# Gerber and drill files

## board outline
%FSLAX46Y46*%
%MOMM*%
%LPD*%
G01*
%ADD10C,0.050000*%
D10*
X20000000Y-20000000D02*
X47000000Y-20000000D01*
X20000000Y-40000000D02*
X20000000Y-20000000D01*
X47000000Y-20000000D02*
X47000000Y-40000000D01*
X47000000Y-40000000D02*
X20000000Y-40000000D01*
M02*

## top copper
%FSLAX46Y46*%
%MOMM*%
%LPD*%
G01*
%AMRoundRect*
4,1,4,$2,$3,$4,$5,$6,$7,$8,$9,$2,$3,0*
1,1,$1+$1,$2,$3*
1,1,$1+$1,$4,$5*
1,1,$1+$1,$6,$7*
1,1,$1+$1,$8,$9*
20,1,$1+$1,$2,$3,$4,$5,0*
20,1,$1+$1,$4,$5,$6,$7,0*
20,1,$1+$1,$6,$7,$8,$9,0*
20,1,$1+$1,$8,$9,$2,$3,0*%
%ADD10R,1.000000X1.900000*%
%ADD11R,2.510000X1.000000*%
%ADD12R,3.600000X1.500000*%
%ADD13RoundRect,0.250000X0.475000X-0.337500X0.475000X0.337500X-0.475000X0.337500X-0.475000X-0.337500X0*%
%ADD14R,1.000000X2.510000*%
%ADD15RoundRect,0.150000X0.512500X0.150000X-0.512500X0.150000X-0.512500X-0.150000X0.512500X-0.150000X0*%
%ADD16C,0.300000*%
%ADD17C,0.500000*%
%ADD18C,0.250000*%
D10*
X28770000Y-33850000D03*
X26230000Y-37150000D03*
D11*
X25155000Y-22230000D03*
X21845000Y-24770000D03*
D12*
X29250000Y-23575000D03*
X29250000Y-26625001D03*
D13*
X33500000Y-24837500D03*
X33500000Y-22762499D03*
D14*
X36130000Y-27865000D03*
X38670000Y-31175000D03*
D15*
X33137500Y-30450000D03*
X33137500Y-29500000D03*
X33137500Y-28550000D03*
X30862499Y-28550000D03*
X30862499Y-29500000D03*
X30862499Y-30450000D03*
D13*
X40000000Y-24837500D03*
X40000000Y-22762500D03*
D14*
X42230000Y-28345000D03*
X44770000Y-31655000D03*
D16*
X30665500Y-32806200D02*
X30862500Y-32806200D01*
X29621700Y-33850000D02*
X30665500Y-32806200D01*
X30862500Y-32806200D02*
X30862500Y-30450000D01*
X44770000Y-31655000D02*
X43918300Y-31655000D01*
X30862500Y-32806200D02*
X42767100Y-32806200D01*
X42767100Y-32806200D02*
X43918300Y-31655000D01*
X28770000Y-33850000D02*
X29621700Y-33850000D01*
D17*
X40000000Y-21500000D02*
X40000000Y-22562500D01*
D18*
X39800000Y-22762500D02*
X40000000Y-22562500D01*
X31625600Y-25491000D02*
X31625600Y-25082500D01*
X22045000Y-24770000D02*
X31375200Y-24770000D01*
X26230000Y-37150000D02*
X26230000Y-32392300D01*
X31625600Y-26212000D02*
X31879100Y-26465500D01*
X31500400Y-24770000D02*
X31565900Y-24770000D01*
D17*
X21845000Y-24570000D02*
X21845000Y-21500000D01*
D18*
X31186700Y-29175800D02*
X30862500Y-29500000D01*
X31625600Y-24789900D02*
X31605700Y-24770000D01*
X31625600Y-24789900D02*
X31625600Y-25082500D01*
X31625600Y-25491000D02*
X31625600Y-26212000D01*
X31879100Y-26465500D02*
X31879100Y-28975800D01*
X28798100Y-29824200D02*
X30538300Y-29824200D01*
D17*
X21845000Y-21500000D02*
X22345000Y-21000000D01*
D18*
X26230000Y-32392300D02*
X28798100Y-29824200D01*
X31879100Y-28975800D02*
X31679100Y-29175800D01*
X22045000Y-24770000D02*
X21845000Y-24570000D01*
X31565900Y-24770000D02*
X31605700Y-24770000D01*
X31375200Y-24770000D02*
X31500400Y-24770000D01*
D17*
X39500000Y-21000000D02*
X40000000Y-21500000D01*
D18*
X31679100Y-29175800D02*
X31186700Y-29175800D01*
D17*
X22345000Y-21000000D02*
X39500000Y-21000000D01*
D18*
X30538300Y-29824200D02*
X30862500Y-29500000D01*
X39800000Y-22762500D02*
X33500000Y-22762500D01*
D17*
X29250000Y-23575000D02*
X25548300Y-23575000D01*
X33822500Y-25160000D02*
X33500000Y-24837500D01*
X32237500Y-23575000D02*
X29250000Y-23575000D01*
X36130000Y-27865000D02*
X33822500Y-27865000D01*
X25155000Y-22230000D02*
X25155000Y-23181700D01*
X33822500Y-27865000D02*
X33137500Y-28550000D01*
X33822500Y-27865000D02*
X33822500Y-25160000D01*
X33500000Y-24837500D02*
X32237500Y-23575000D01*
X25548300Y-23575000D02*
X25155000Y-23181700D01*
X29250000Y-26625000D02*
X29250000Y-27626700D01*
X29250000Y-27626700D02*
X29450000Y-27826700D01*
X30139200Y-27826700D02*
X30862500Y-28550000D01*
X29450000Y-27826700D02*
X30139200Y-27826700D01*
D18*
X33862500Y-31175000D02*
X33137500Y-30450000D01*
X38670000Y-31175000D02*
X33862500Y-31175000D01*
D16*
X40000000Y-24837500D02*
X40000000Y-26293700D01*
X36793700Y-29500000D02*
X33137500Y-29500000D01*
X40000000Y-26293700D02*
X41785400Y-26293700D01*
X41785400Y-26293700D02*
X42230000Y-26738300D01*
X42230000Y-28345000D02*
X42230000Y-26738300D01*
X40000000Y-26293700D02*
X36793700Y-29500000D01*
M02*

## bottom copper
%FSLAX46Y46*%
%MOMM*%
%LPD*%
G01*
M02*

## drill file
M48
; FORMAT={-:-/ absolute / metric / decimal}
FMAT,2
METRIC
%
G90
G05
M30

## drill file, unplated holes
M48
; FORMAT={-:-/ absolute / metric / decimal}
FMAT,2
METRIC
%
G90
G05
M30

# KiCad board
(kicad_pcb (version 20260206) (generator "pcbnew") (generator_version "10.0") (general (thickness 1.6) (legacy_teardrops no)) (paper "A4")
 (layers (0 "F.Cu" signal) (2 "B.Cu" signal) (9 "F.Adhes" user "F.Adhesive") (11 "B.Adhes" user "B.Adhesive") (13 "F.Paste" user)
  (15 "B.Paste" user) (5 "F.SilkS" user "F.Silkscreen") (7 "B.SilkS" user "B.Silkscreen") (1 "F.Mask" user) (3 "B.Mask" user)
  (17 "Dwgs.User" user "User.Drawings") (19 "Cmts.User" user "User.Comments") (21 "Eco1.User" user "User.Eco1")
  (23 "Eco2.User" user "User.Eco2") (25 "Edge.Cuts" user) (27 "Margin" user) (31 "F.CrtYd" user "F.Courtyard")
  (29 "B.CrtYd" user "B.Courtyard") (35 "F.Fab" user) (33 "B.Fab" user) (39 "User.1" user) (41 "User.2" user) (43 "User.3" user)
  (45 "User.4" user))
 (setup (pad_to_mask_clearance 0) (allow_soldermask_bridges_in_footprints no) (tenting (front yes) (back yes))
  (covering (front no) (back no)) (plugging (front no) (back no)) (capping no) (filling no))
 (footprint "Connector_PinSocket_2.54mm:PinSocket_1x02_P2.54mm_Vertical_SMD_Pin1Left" (layer "F.Cu") (at 27.5 35.5 -90)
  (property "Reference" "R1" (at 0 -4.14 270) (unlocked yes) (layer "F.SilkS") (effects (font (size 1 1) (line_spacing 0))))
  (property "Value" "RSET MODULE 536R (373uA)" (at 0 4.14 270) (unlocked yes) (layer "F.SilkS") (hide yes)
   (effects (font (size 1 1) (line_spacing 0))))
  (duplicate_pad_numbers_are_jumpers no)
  (pad "1" smd rect (at -1.65 -1.27 270) (size 1.9 1) (layers "F.Cu" "F.Mask" "F.Paste") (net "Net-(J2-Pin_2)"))
  (pad "2" smd rect (at 1.65 1.27 270) (size 1.9 1) (layers "F.Cu" "F.Mask" "F.Paste") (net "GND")))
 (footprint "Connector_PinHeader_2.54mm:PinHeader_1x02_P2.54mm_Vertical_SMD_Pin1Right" (layer "F.Cu") (at 23.5 23.5)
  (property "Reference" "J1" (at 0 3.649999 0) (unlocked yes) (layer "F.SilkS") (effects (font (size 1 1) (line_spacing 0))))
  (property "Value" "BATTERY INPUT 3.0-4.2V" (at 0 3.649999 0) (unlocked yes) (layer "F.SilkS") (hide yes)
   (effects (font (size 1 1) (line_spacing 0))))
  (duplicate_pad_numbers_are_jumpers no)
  (pad "1" smd rect (at 1.655 -1.27) (size 2.51 1) (layers "F.Cu" "F.Mask" "F.Paste") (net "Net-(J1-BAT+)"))
  (pad "2" smd rect (at -1.655 1.27) (size 2.51 1) (layers "F.Cu" "F.Mask" "F.Paste") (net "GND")))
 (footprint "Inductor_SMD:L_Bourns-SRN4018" (layer "F.Cu") (at 29.25 25.1 -90)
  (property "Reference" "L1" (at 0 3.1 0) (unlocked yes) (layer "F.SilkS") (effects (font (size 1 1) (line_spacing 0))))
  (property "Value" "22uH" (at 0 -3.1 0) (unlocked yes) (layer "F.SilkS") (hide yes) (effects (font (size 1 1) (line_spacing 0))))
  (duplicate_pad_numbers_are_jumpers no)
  (pad "1" smd rect (at -1.525 0 270) (size 1.5 3.6) (layers "F.Cu" "F.Mask" "F.Paste") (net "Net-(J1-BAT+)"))
  (pad "2" smd rect (at 1.525001 0 270) (size 1.5 3.6) (layers "F.Cu" "F.Mask" "F.Paste") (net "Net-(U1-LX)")))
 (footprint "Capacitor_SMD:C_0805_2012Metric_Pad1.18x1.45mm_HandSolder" (layer "F.Cu") (at 33.5 23.8 90)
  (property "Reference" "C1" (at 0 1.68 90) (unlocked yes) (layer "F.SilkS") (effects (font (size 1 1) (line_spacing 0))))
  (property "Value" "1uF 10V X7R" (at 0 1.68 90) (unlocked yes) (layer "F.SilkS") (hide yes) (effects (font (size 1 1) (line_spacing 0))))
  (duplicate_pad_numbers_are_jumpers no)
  (pad "1" smd roundrect (at -1.0375 0 90) (size 1.175 1.45) (layers "F.Cu" "F.Mask" "F.Paste") (roundrect_rratio 0.212766)
   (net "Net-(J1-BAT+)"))
  (pad "2" smd roundrect (at 1.037501 0 90) (size 1.175 1.45) (layers "F.Cu" "F.Mask" "F.Paste") (roundrect_rratio 0.212766) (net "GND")
   (zone_connect 3)))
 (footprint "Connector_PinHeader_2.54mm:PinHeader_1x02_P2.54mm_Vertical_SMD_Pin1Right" (layer "F.Cu") (at 37.4 29.52 90)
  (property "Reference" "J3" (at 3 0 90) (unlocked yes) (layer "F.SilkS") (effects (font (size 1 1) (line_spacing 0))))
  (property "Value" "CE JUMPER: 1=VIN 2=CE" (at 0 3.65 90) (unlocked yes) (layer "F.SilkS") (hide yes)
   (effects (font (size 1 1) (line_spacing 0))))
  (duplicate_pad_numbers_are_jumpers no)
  (pad "1" smd rect (at 1.655 -1.27 90) (size 2.51 1) (layers "F.Cu" "F.Mask" "F.Paste") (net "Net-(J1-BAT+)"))
  (pad "2" smd rect (at -1.655 1.27 90) (size 2.51 1) (layers "F.Cu" "F.Mask" "F.Paste") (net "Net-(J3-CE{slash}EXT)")))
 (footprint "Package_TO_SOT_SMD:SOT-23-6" (layer "F.Cu") (at 32 29.5 180)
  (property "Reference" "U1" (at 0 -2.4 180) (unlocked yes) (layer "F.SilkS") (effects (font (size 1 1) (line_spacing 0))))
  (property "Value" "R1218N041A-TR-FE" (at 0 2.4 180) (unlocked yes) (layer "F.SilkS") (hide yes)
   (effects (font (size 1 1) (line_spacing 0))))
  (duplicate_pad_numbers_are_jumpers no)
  (pad "1" smd roundrect (at -1.1375 -0.95 180) (size 1.325 0.6) (layers "F.Cu" "F.Mask" "F.Paste") (roundrect_rratio 0.25)
   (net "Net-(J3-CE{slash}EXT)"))
  (pad "2" smd roundrect (at -1.1375 0 180) (size 1.325 0.6) (layers "F.Cu" "F.Mask" "F.Paste") (roundrect_rratio 0.25)
   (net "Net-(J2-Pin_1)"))
  (pad "3" smd roundrect (at -1.1375 0.95 180) (size 1.325 0.6) (layers "F.Cu" "F.Mask" "F.Paste") (roundrect_rratio 0.25)
   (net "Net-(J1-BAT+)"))
  (pad "4" smd roundrect (at 1.137501 0.95 180) (size 1.325 0.6) (layers "F.Cu" "F.Mask" "F.Paste") (roundrect_rratio 0.25)
   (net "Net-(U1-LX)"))
  (pad "5" smd roundrect (at 1.137501 0 180) (size 1.325 0.6) (layers "F.Cu" "F.Mask" "F.Paste") (roundrect_rratio 0.25) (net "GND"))
  (pad "6" smd roundrect (at 1.137501 -0.95 180) (size 1.325 0.6) (layers "F.Cu" "F.Mask" "F.Paste") (roundrect_rratio 0.25)
   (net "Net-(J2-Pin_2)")))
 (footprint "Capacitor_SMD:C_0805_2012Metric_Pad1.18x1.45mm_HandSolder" (layer "F.Cu") (at 40 23.8 90)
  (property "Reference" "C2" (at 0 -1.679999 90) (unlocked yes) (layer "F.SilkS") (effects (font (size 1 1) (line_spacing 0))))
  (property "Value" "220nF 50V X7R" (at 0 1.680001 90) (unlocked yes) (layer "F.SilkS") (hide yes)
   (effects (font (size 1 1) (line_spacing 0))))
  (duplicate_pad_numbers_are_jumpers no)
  (pad "1" smd roundrect (at -1.0375 0 90) (size 1.175 1.45) (layers "F.Cu" "F.Mask" "F.Paste") (roundrect_rratio 0.212766)
   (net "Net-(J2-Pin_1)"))
  (pad "2" smd roundrect (at 1.0375 0 90) (size 1.175 1.45) (layers "F.Cu" "F.Mask" "F.Paste") (roundrect_rratio 0.212766) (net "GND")
   (zone_connect 3)))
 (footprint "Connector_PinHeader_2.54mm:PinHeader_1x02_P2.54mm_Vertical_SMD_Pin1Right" (layer "F.Cu") (at 43.5 30 90)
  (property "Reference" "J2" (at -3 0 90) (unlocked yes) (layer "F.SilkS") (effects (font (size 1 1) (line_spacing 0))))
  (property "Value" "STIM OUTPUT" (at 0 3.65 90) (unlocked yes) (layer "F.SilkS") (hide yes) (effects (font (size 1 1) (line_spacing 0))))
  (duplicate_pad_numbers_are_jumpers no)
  (pad "1" smd rect (at 1.655 -1.27 90) (size 2.51 1) (layers "F.Cu" "F.Mask" "F.Paste") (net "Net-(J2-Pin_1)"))
  (pad "2" smd rect (at -1.655 1.27 90) (size 2.51 1) (layers "F.Cu" "F.Mask" "F.Paste") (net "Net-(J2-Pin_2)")))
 (gr_line (start 20 20) (end 47 20) (stroke (width 0.05) (type default)) (layer "Edge.Cuts"))
 (gr_line (start 20 40) (end 20 20) (stroke (width 0.05) (type default)) (layer "Edge.Cuts"))
 (gr_line (start 47 20) (end 47 40) (stroke (width 0.05) (type default)) (layer "Edge.Cuts"))
 (gr_line (start 47 40) (end 20 40) (stroke (width 0.05) (type default)) (layer "Edge.Cuts"))
 (segment (start 30.6655 32.8062) (end 30.8625 32.8062) (width 0.3) (layer "F.Cu") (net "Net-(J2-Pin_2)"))
 (segment (start 29.6217 33.85) (end 30.6655 32.8062) (width 0.3) (layer "F.Cu") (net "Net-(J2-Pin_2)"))
 (segment (start 30.8625 32.8062) (end 30.8625 30.45) (width 0.3) (layer "F.Cu") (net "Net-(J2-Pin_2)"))
 (segment (start 44.77 31.655) (end 43.9183 31.655) (width 0.3) (layer "F.Cu") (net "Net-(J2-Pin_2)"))
 (segment (start 30.8625 32.8062) (end 42.7671 32.8062) (width 0.3) (layer "F.Cu") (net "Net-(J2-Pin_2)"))
 (segment (start 42.7671 32.8062) (end 43.9183 31.655) (width 0.3) (layer "F.Cu") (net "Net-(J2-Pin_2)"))
 (segment (start 28.77 33.85) (end 29.6217 33.85) (width 0.3) (layer "F.Cu") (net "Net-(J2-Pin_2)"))
 (segment (start 31.6256 25.491) (end 31.6256 25.0825) (width 0.25) (layer "F.Cu") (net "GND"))
 (segment (start 22.045000 24.770000) (end 31.3752 24.77) (width 0.25) (layer "F.Cu") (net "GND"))
 (segment (start 26.23 37.15) (end 26.23 32.3923) (width 0.25) (layer "F.Cu") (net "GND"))
 (segment (start 31.6256 26.212) (end 31.8791 26.4655) (width 0.25) (layer "F.Cu") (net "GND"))
 (segment (start 31.5004 24.77) (end 31.5659 24.77) (width 0.25) (layer "F.Cu") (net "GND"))
 (segment (start 31.1867 29.1758) (end 30.8625 29.5) (width 0.25) (layer "F.Cu") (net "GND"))
 (segment (start 31.625600 24.789900) (end 31.6256 25.0825) (width 0.25) (layer "F.Cu") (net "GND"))
 (segment (start 31.6256 25.491) (end 31.6256 26.212) (width 0.25) (layer "F.Cu") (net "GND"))
 (segment (start 31.8791 26.4655) (end 31.879100 28.975800) (width 0.25) (layer "F.Cu") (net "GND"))
 (segment (start 28.7981 29.8242) (end 30.5383 29.8242) (width 0.25) (layer "F.Cu") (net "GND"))
 (segment (start 26.23 32.3923) (end 28.7981 29.8242) (width 0.25) (layer "F.Cu") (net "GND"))
 (segment (start 31.5659 24.77) (end 31.605700 24.770000) (width 0.25) (layer "F.Cu") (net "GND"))
 (segment (start 31.3752 24.77) (end 31.5004 24.77) (width 0.25) (layer "F.Cu") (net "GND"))
 (segment (start 31.679100 29.175800) (end 31.1867 29.1758) (width 0.25) (layer "F.Cu") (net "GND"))
 (segment (start 30.5383 29.8242) (end 30.8625 29.5) (width 0.25) (layer "F.Cu") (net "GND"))
 (segment (start 39.800000 22.762500) (end 33.5 22.7625) (width 0.25) (layer "F.Cu") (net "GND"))
 (segment (start 29.25 23.575) (end 25.5483 23.575) (width 0.5) (layer "F.Cu") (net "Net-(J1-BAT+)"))
 (segment (start 33.8225 25.16) (end 33.5 24.8375) (width 0.5) (layer "F.Cu") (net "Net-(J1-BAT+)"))
 (segment (start 32.2375 23.575) (end 29.25 23.575) (width 0.5) (layer "F.Cu") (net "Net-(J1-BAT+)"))
 (segment (start 36.13 27.865) (end 33.8225 27.865) (width 0.5) (layer "F.Cu") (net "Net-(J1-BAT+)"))
 (segment (start 25.155 22.23) (end 25.155 23.1817) (width 0.5) (layer "F.Cu") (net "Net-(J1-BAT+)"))
 (segment (start 33.8225 27.865) (end 33.1375 28.55) (width 0.5) (layer "F.Cu") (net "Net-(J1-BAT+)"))
 (segment (start 33.8225 27.865) (end 33.8225 25.16) (width 0.5) (layer "F.Cu") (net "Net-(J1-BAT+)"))
 (segment (start 33.5 24.8375) (end 32.2375 23.575) (width 0.5) (layer "F.Cu") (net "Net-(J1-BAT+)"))
 (segment (start 25.5483 23.575) (end 25.155 23.1817) (width 0.5) (layer "F.Cu") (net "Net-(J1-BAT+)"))
 (segment (start 29.25 26.625) (end 29.250000 27.626700) (width 0.5) (layer "F.Cu") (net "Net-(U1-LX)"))
 (segment (start 30.1392 27.8267) (end 30.8625 28.55) (width 0.5) (layer "F.Cu") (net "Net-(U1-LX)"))
 (segment (start 29.450000 27.826700) (end 30.1392 27.8267) (width 0.5) (layer "F.Cu") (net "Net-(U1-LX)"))
 (segment (start 33.8625 31.175) (end 33.1375 30.45) (width 0.25) (layer "F.Cu") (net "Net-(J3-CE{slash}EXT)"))
 (segment (start 38.67 31.175) (end 33.8625 31.175) (width 0.25) (layer "F.Cu") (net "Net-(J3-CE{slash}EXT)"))
 (segment (start 40 24.8375) (end 40 26.2937) (width 0.3) (layer "F.Cu") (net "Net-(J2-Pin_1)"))
 (segment (start 36.7937 29.5) (end 33.1375 29.5) (width 0.3) (layer "F.Cu") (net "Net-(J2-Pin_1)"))
 (segment (start 40 26.2937) (end 41.7854 26.2937) (width 0.3) (layer "F.Cu") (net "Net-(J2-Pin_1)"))
 (segment (start 41.7854 26.2937) (end 42.23 26.7383) (width 0.3) (layer "F.Cu") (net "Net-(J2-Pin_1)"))
 (segment (start 42.23 28.345) (end 42.23 26.7383) (width 0.3) (layer "F.Cu") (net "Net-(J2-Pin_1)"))
 (segment (start 40 26.2937) (end 36.7937 29.5) (width 0.3) (layer "F.Cu") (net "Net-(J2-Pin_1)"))
 (segment (start 31.625600 24.789900) (end 31.605700 24.770000) (width 0.25) (layer "F.Cu") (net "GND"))
 (segment (start 31.879100 28.975800) (end 31.679100 29.175800) (width 0.25) (layer "F.Cu") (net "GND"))
 (segment (start 29.250000 27.626700) (end 29.450000 27.826700) (width 0.5) (layer "F.Cu") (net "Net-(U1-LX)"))
 (segment (start 21.845000 24.570000) (end 21.845 21.5) (width 0.5) (layer "F.Cu") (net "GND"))
 (segment (start 21.845 21.5) (end 22.345 21.0) (width 0.5) (layer "F.Cu") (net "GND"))
 (segment (start 22.345 21.0) (end 39.5 21.0) (width 0.5) (layer "F.Cu") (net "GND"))
 (segment (start 39.5 21.0) (end 40.0 21.5) (width 0.5) (layer "F.Cu") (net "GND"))
 (segment (start 40.0 21.5) (end 40.000000 22.562500) (width 0.5) (layer "F.Cu") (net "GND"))
 (segment (start 22.045000 24.770000) (end 21.845000 24.570000) (width 0.25) (layer "F.Cu") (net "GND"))
 (segment (start 39.800000 22.762500) (end 40.000000 22.562500) (width 0.25) (layer "F.Cu") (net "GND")))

